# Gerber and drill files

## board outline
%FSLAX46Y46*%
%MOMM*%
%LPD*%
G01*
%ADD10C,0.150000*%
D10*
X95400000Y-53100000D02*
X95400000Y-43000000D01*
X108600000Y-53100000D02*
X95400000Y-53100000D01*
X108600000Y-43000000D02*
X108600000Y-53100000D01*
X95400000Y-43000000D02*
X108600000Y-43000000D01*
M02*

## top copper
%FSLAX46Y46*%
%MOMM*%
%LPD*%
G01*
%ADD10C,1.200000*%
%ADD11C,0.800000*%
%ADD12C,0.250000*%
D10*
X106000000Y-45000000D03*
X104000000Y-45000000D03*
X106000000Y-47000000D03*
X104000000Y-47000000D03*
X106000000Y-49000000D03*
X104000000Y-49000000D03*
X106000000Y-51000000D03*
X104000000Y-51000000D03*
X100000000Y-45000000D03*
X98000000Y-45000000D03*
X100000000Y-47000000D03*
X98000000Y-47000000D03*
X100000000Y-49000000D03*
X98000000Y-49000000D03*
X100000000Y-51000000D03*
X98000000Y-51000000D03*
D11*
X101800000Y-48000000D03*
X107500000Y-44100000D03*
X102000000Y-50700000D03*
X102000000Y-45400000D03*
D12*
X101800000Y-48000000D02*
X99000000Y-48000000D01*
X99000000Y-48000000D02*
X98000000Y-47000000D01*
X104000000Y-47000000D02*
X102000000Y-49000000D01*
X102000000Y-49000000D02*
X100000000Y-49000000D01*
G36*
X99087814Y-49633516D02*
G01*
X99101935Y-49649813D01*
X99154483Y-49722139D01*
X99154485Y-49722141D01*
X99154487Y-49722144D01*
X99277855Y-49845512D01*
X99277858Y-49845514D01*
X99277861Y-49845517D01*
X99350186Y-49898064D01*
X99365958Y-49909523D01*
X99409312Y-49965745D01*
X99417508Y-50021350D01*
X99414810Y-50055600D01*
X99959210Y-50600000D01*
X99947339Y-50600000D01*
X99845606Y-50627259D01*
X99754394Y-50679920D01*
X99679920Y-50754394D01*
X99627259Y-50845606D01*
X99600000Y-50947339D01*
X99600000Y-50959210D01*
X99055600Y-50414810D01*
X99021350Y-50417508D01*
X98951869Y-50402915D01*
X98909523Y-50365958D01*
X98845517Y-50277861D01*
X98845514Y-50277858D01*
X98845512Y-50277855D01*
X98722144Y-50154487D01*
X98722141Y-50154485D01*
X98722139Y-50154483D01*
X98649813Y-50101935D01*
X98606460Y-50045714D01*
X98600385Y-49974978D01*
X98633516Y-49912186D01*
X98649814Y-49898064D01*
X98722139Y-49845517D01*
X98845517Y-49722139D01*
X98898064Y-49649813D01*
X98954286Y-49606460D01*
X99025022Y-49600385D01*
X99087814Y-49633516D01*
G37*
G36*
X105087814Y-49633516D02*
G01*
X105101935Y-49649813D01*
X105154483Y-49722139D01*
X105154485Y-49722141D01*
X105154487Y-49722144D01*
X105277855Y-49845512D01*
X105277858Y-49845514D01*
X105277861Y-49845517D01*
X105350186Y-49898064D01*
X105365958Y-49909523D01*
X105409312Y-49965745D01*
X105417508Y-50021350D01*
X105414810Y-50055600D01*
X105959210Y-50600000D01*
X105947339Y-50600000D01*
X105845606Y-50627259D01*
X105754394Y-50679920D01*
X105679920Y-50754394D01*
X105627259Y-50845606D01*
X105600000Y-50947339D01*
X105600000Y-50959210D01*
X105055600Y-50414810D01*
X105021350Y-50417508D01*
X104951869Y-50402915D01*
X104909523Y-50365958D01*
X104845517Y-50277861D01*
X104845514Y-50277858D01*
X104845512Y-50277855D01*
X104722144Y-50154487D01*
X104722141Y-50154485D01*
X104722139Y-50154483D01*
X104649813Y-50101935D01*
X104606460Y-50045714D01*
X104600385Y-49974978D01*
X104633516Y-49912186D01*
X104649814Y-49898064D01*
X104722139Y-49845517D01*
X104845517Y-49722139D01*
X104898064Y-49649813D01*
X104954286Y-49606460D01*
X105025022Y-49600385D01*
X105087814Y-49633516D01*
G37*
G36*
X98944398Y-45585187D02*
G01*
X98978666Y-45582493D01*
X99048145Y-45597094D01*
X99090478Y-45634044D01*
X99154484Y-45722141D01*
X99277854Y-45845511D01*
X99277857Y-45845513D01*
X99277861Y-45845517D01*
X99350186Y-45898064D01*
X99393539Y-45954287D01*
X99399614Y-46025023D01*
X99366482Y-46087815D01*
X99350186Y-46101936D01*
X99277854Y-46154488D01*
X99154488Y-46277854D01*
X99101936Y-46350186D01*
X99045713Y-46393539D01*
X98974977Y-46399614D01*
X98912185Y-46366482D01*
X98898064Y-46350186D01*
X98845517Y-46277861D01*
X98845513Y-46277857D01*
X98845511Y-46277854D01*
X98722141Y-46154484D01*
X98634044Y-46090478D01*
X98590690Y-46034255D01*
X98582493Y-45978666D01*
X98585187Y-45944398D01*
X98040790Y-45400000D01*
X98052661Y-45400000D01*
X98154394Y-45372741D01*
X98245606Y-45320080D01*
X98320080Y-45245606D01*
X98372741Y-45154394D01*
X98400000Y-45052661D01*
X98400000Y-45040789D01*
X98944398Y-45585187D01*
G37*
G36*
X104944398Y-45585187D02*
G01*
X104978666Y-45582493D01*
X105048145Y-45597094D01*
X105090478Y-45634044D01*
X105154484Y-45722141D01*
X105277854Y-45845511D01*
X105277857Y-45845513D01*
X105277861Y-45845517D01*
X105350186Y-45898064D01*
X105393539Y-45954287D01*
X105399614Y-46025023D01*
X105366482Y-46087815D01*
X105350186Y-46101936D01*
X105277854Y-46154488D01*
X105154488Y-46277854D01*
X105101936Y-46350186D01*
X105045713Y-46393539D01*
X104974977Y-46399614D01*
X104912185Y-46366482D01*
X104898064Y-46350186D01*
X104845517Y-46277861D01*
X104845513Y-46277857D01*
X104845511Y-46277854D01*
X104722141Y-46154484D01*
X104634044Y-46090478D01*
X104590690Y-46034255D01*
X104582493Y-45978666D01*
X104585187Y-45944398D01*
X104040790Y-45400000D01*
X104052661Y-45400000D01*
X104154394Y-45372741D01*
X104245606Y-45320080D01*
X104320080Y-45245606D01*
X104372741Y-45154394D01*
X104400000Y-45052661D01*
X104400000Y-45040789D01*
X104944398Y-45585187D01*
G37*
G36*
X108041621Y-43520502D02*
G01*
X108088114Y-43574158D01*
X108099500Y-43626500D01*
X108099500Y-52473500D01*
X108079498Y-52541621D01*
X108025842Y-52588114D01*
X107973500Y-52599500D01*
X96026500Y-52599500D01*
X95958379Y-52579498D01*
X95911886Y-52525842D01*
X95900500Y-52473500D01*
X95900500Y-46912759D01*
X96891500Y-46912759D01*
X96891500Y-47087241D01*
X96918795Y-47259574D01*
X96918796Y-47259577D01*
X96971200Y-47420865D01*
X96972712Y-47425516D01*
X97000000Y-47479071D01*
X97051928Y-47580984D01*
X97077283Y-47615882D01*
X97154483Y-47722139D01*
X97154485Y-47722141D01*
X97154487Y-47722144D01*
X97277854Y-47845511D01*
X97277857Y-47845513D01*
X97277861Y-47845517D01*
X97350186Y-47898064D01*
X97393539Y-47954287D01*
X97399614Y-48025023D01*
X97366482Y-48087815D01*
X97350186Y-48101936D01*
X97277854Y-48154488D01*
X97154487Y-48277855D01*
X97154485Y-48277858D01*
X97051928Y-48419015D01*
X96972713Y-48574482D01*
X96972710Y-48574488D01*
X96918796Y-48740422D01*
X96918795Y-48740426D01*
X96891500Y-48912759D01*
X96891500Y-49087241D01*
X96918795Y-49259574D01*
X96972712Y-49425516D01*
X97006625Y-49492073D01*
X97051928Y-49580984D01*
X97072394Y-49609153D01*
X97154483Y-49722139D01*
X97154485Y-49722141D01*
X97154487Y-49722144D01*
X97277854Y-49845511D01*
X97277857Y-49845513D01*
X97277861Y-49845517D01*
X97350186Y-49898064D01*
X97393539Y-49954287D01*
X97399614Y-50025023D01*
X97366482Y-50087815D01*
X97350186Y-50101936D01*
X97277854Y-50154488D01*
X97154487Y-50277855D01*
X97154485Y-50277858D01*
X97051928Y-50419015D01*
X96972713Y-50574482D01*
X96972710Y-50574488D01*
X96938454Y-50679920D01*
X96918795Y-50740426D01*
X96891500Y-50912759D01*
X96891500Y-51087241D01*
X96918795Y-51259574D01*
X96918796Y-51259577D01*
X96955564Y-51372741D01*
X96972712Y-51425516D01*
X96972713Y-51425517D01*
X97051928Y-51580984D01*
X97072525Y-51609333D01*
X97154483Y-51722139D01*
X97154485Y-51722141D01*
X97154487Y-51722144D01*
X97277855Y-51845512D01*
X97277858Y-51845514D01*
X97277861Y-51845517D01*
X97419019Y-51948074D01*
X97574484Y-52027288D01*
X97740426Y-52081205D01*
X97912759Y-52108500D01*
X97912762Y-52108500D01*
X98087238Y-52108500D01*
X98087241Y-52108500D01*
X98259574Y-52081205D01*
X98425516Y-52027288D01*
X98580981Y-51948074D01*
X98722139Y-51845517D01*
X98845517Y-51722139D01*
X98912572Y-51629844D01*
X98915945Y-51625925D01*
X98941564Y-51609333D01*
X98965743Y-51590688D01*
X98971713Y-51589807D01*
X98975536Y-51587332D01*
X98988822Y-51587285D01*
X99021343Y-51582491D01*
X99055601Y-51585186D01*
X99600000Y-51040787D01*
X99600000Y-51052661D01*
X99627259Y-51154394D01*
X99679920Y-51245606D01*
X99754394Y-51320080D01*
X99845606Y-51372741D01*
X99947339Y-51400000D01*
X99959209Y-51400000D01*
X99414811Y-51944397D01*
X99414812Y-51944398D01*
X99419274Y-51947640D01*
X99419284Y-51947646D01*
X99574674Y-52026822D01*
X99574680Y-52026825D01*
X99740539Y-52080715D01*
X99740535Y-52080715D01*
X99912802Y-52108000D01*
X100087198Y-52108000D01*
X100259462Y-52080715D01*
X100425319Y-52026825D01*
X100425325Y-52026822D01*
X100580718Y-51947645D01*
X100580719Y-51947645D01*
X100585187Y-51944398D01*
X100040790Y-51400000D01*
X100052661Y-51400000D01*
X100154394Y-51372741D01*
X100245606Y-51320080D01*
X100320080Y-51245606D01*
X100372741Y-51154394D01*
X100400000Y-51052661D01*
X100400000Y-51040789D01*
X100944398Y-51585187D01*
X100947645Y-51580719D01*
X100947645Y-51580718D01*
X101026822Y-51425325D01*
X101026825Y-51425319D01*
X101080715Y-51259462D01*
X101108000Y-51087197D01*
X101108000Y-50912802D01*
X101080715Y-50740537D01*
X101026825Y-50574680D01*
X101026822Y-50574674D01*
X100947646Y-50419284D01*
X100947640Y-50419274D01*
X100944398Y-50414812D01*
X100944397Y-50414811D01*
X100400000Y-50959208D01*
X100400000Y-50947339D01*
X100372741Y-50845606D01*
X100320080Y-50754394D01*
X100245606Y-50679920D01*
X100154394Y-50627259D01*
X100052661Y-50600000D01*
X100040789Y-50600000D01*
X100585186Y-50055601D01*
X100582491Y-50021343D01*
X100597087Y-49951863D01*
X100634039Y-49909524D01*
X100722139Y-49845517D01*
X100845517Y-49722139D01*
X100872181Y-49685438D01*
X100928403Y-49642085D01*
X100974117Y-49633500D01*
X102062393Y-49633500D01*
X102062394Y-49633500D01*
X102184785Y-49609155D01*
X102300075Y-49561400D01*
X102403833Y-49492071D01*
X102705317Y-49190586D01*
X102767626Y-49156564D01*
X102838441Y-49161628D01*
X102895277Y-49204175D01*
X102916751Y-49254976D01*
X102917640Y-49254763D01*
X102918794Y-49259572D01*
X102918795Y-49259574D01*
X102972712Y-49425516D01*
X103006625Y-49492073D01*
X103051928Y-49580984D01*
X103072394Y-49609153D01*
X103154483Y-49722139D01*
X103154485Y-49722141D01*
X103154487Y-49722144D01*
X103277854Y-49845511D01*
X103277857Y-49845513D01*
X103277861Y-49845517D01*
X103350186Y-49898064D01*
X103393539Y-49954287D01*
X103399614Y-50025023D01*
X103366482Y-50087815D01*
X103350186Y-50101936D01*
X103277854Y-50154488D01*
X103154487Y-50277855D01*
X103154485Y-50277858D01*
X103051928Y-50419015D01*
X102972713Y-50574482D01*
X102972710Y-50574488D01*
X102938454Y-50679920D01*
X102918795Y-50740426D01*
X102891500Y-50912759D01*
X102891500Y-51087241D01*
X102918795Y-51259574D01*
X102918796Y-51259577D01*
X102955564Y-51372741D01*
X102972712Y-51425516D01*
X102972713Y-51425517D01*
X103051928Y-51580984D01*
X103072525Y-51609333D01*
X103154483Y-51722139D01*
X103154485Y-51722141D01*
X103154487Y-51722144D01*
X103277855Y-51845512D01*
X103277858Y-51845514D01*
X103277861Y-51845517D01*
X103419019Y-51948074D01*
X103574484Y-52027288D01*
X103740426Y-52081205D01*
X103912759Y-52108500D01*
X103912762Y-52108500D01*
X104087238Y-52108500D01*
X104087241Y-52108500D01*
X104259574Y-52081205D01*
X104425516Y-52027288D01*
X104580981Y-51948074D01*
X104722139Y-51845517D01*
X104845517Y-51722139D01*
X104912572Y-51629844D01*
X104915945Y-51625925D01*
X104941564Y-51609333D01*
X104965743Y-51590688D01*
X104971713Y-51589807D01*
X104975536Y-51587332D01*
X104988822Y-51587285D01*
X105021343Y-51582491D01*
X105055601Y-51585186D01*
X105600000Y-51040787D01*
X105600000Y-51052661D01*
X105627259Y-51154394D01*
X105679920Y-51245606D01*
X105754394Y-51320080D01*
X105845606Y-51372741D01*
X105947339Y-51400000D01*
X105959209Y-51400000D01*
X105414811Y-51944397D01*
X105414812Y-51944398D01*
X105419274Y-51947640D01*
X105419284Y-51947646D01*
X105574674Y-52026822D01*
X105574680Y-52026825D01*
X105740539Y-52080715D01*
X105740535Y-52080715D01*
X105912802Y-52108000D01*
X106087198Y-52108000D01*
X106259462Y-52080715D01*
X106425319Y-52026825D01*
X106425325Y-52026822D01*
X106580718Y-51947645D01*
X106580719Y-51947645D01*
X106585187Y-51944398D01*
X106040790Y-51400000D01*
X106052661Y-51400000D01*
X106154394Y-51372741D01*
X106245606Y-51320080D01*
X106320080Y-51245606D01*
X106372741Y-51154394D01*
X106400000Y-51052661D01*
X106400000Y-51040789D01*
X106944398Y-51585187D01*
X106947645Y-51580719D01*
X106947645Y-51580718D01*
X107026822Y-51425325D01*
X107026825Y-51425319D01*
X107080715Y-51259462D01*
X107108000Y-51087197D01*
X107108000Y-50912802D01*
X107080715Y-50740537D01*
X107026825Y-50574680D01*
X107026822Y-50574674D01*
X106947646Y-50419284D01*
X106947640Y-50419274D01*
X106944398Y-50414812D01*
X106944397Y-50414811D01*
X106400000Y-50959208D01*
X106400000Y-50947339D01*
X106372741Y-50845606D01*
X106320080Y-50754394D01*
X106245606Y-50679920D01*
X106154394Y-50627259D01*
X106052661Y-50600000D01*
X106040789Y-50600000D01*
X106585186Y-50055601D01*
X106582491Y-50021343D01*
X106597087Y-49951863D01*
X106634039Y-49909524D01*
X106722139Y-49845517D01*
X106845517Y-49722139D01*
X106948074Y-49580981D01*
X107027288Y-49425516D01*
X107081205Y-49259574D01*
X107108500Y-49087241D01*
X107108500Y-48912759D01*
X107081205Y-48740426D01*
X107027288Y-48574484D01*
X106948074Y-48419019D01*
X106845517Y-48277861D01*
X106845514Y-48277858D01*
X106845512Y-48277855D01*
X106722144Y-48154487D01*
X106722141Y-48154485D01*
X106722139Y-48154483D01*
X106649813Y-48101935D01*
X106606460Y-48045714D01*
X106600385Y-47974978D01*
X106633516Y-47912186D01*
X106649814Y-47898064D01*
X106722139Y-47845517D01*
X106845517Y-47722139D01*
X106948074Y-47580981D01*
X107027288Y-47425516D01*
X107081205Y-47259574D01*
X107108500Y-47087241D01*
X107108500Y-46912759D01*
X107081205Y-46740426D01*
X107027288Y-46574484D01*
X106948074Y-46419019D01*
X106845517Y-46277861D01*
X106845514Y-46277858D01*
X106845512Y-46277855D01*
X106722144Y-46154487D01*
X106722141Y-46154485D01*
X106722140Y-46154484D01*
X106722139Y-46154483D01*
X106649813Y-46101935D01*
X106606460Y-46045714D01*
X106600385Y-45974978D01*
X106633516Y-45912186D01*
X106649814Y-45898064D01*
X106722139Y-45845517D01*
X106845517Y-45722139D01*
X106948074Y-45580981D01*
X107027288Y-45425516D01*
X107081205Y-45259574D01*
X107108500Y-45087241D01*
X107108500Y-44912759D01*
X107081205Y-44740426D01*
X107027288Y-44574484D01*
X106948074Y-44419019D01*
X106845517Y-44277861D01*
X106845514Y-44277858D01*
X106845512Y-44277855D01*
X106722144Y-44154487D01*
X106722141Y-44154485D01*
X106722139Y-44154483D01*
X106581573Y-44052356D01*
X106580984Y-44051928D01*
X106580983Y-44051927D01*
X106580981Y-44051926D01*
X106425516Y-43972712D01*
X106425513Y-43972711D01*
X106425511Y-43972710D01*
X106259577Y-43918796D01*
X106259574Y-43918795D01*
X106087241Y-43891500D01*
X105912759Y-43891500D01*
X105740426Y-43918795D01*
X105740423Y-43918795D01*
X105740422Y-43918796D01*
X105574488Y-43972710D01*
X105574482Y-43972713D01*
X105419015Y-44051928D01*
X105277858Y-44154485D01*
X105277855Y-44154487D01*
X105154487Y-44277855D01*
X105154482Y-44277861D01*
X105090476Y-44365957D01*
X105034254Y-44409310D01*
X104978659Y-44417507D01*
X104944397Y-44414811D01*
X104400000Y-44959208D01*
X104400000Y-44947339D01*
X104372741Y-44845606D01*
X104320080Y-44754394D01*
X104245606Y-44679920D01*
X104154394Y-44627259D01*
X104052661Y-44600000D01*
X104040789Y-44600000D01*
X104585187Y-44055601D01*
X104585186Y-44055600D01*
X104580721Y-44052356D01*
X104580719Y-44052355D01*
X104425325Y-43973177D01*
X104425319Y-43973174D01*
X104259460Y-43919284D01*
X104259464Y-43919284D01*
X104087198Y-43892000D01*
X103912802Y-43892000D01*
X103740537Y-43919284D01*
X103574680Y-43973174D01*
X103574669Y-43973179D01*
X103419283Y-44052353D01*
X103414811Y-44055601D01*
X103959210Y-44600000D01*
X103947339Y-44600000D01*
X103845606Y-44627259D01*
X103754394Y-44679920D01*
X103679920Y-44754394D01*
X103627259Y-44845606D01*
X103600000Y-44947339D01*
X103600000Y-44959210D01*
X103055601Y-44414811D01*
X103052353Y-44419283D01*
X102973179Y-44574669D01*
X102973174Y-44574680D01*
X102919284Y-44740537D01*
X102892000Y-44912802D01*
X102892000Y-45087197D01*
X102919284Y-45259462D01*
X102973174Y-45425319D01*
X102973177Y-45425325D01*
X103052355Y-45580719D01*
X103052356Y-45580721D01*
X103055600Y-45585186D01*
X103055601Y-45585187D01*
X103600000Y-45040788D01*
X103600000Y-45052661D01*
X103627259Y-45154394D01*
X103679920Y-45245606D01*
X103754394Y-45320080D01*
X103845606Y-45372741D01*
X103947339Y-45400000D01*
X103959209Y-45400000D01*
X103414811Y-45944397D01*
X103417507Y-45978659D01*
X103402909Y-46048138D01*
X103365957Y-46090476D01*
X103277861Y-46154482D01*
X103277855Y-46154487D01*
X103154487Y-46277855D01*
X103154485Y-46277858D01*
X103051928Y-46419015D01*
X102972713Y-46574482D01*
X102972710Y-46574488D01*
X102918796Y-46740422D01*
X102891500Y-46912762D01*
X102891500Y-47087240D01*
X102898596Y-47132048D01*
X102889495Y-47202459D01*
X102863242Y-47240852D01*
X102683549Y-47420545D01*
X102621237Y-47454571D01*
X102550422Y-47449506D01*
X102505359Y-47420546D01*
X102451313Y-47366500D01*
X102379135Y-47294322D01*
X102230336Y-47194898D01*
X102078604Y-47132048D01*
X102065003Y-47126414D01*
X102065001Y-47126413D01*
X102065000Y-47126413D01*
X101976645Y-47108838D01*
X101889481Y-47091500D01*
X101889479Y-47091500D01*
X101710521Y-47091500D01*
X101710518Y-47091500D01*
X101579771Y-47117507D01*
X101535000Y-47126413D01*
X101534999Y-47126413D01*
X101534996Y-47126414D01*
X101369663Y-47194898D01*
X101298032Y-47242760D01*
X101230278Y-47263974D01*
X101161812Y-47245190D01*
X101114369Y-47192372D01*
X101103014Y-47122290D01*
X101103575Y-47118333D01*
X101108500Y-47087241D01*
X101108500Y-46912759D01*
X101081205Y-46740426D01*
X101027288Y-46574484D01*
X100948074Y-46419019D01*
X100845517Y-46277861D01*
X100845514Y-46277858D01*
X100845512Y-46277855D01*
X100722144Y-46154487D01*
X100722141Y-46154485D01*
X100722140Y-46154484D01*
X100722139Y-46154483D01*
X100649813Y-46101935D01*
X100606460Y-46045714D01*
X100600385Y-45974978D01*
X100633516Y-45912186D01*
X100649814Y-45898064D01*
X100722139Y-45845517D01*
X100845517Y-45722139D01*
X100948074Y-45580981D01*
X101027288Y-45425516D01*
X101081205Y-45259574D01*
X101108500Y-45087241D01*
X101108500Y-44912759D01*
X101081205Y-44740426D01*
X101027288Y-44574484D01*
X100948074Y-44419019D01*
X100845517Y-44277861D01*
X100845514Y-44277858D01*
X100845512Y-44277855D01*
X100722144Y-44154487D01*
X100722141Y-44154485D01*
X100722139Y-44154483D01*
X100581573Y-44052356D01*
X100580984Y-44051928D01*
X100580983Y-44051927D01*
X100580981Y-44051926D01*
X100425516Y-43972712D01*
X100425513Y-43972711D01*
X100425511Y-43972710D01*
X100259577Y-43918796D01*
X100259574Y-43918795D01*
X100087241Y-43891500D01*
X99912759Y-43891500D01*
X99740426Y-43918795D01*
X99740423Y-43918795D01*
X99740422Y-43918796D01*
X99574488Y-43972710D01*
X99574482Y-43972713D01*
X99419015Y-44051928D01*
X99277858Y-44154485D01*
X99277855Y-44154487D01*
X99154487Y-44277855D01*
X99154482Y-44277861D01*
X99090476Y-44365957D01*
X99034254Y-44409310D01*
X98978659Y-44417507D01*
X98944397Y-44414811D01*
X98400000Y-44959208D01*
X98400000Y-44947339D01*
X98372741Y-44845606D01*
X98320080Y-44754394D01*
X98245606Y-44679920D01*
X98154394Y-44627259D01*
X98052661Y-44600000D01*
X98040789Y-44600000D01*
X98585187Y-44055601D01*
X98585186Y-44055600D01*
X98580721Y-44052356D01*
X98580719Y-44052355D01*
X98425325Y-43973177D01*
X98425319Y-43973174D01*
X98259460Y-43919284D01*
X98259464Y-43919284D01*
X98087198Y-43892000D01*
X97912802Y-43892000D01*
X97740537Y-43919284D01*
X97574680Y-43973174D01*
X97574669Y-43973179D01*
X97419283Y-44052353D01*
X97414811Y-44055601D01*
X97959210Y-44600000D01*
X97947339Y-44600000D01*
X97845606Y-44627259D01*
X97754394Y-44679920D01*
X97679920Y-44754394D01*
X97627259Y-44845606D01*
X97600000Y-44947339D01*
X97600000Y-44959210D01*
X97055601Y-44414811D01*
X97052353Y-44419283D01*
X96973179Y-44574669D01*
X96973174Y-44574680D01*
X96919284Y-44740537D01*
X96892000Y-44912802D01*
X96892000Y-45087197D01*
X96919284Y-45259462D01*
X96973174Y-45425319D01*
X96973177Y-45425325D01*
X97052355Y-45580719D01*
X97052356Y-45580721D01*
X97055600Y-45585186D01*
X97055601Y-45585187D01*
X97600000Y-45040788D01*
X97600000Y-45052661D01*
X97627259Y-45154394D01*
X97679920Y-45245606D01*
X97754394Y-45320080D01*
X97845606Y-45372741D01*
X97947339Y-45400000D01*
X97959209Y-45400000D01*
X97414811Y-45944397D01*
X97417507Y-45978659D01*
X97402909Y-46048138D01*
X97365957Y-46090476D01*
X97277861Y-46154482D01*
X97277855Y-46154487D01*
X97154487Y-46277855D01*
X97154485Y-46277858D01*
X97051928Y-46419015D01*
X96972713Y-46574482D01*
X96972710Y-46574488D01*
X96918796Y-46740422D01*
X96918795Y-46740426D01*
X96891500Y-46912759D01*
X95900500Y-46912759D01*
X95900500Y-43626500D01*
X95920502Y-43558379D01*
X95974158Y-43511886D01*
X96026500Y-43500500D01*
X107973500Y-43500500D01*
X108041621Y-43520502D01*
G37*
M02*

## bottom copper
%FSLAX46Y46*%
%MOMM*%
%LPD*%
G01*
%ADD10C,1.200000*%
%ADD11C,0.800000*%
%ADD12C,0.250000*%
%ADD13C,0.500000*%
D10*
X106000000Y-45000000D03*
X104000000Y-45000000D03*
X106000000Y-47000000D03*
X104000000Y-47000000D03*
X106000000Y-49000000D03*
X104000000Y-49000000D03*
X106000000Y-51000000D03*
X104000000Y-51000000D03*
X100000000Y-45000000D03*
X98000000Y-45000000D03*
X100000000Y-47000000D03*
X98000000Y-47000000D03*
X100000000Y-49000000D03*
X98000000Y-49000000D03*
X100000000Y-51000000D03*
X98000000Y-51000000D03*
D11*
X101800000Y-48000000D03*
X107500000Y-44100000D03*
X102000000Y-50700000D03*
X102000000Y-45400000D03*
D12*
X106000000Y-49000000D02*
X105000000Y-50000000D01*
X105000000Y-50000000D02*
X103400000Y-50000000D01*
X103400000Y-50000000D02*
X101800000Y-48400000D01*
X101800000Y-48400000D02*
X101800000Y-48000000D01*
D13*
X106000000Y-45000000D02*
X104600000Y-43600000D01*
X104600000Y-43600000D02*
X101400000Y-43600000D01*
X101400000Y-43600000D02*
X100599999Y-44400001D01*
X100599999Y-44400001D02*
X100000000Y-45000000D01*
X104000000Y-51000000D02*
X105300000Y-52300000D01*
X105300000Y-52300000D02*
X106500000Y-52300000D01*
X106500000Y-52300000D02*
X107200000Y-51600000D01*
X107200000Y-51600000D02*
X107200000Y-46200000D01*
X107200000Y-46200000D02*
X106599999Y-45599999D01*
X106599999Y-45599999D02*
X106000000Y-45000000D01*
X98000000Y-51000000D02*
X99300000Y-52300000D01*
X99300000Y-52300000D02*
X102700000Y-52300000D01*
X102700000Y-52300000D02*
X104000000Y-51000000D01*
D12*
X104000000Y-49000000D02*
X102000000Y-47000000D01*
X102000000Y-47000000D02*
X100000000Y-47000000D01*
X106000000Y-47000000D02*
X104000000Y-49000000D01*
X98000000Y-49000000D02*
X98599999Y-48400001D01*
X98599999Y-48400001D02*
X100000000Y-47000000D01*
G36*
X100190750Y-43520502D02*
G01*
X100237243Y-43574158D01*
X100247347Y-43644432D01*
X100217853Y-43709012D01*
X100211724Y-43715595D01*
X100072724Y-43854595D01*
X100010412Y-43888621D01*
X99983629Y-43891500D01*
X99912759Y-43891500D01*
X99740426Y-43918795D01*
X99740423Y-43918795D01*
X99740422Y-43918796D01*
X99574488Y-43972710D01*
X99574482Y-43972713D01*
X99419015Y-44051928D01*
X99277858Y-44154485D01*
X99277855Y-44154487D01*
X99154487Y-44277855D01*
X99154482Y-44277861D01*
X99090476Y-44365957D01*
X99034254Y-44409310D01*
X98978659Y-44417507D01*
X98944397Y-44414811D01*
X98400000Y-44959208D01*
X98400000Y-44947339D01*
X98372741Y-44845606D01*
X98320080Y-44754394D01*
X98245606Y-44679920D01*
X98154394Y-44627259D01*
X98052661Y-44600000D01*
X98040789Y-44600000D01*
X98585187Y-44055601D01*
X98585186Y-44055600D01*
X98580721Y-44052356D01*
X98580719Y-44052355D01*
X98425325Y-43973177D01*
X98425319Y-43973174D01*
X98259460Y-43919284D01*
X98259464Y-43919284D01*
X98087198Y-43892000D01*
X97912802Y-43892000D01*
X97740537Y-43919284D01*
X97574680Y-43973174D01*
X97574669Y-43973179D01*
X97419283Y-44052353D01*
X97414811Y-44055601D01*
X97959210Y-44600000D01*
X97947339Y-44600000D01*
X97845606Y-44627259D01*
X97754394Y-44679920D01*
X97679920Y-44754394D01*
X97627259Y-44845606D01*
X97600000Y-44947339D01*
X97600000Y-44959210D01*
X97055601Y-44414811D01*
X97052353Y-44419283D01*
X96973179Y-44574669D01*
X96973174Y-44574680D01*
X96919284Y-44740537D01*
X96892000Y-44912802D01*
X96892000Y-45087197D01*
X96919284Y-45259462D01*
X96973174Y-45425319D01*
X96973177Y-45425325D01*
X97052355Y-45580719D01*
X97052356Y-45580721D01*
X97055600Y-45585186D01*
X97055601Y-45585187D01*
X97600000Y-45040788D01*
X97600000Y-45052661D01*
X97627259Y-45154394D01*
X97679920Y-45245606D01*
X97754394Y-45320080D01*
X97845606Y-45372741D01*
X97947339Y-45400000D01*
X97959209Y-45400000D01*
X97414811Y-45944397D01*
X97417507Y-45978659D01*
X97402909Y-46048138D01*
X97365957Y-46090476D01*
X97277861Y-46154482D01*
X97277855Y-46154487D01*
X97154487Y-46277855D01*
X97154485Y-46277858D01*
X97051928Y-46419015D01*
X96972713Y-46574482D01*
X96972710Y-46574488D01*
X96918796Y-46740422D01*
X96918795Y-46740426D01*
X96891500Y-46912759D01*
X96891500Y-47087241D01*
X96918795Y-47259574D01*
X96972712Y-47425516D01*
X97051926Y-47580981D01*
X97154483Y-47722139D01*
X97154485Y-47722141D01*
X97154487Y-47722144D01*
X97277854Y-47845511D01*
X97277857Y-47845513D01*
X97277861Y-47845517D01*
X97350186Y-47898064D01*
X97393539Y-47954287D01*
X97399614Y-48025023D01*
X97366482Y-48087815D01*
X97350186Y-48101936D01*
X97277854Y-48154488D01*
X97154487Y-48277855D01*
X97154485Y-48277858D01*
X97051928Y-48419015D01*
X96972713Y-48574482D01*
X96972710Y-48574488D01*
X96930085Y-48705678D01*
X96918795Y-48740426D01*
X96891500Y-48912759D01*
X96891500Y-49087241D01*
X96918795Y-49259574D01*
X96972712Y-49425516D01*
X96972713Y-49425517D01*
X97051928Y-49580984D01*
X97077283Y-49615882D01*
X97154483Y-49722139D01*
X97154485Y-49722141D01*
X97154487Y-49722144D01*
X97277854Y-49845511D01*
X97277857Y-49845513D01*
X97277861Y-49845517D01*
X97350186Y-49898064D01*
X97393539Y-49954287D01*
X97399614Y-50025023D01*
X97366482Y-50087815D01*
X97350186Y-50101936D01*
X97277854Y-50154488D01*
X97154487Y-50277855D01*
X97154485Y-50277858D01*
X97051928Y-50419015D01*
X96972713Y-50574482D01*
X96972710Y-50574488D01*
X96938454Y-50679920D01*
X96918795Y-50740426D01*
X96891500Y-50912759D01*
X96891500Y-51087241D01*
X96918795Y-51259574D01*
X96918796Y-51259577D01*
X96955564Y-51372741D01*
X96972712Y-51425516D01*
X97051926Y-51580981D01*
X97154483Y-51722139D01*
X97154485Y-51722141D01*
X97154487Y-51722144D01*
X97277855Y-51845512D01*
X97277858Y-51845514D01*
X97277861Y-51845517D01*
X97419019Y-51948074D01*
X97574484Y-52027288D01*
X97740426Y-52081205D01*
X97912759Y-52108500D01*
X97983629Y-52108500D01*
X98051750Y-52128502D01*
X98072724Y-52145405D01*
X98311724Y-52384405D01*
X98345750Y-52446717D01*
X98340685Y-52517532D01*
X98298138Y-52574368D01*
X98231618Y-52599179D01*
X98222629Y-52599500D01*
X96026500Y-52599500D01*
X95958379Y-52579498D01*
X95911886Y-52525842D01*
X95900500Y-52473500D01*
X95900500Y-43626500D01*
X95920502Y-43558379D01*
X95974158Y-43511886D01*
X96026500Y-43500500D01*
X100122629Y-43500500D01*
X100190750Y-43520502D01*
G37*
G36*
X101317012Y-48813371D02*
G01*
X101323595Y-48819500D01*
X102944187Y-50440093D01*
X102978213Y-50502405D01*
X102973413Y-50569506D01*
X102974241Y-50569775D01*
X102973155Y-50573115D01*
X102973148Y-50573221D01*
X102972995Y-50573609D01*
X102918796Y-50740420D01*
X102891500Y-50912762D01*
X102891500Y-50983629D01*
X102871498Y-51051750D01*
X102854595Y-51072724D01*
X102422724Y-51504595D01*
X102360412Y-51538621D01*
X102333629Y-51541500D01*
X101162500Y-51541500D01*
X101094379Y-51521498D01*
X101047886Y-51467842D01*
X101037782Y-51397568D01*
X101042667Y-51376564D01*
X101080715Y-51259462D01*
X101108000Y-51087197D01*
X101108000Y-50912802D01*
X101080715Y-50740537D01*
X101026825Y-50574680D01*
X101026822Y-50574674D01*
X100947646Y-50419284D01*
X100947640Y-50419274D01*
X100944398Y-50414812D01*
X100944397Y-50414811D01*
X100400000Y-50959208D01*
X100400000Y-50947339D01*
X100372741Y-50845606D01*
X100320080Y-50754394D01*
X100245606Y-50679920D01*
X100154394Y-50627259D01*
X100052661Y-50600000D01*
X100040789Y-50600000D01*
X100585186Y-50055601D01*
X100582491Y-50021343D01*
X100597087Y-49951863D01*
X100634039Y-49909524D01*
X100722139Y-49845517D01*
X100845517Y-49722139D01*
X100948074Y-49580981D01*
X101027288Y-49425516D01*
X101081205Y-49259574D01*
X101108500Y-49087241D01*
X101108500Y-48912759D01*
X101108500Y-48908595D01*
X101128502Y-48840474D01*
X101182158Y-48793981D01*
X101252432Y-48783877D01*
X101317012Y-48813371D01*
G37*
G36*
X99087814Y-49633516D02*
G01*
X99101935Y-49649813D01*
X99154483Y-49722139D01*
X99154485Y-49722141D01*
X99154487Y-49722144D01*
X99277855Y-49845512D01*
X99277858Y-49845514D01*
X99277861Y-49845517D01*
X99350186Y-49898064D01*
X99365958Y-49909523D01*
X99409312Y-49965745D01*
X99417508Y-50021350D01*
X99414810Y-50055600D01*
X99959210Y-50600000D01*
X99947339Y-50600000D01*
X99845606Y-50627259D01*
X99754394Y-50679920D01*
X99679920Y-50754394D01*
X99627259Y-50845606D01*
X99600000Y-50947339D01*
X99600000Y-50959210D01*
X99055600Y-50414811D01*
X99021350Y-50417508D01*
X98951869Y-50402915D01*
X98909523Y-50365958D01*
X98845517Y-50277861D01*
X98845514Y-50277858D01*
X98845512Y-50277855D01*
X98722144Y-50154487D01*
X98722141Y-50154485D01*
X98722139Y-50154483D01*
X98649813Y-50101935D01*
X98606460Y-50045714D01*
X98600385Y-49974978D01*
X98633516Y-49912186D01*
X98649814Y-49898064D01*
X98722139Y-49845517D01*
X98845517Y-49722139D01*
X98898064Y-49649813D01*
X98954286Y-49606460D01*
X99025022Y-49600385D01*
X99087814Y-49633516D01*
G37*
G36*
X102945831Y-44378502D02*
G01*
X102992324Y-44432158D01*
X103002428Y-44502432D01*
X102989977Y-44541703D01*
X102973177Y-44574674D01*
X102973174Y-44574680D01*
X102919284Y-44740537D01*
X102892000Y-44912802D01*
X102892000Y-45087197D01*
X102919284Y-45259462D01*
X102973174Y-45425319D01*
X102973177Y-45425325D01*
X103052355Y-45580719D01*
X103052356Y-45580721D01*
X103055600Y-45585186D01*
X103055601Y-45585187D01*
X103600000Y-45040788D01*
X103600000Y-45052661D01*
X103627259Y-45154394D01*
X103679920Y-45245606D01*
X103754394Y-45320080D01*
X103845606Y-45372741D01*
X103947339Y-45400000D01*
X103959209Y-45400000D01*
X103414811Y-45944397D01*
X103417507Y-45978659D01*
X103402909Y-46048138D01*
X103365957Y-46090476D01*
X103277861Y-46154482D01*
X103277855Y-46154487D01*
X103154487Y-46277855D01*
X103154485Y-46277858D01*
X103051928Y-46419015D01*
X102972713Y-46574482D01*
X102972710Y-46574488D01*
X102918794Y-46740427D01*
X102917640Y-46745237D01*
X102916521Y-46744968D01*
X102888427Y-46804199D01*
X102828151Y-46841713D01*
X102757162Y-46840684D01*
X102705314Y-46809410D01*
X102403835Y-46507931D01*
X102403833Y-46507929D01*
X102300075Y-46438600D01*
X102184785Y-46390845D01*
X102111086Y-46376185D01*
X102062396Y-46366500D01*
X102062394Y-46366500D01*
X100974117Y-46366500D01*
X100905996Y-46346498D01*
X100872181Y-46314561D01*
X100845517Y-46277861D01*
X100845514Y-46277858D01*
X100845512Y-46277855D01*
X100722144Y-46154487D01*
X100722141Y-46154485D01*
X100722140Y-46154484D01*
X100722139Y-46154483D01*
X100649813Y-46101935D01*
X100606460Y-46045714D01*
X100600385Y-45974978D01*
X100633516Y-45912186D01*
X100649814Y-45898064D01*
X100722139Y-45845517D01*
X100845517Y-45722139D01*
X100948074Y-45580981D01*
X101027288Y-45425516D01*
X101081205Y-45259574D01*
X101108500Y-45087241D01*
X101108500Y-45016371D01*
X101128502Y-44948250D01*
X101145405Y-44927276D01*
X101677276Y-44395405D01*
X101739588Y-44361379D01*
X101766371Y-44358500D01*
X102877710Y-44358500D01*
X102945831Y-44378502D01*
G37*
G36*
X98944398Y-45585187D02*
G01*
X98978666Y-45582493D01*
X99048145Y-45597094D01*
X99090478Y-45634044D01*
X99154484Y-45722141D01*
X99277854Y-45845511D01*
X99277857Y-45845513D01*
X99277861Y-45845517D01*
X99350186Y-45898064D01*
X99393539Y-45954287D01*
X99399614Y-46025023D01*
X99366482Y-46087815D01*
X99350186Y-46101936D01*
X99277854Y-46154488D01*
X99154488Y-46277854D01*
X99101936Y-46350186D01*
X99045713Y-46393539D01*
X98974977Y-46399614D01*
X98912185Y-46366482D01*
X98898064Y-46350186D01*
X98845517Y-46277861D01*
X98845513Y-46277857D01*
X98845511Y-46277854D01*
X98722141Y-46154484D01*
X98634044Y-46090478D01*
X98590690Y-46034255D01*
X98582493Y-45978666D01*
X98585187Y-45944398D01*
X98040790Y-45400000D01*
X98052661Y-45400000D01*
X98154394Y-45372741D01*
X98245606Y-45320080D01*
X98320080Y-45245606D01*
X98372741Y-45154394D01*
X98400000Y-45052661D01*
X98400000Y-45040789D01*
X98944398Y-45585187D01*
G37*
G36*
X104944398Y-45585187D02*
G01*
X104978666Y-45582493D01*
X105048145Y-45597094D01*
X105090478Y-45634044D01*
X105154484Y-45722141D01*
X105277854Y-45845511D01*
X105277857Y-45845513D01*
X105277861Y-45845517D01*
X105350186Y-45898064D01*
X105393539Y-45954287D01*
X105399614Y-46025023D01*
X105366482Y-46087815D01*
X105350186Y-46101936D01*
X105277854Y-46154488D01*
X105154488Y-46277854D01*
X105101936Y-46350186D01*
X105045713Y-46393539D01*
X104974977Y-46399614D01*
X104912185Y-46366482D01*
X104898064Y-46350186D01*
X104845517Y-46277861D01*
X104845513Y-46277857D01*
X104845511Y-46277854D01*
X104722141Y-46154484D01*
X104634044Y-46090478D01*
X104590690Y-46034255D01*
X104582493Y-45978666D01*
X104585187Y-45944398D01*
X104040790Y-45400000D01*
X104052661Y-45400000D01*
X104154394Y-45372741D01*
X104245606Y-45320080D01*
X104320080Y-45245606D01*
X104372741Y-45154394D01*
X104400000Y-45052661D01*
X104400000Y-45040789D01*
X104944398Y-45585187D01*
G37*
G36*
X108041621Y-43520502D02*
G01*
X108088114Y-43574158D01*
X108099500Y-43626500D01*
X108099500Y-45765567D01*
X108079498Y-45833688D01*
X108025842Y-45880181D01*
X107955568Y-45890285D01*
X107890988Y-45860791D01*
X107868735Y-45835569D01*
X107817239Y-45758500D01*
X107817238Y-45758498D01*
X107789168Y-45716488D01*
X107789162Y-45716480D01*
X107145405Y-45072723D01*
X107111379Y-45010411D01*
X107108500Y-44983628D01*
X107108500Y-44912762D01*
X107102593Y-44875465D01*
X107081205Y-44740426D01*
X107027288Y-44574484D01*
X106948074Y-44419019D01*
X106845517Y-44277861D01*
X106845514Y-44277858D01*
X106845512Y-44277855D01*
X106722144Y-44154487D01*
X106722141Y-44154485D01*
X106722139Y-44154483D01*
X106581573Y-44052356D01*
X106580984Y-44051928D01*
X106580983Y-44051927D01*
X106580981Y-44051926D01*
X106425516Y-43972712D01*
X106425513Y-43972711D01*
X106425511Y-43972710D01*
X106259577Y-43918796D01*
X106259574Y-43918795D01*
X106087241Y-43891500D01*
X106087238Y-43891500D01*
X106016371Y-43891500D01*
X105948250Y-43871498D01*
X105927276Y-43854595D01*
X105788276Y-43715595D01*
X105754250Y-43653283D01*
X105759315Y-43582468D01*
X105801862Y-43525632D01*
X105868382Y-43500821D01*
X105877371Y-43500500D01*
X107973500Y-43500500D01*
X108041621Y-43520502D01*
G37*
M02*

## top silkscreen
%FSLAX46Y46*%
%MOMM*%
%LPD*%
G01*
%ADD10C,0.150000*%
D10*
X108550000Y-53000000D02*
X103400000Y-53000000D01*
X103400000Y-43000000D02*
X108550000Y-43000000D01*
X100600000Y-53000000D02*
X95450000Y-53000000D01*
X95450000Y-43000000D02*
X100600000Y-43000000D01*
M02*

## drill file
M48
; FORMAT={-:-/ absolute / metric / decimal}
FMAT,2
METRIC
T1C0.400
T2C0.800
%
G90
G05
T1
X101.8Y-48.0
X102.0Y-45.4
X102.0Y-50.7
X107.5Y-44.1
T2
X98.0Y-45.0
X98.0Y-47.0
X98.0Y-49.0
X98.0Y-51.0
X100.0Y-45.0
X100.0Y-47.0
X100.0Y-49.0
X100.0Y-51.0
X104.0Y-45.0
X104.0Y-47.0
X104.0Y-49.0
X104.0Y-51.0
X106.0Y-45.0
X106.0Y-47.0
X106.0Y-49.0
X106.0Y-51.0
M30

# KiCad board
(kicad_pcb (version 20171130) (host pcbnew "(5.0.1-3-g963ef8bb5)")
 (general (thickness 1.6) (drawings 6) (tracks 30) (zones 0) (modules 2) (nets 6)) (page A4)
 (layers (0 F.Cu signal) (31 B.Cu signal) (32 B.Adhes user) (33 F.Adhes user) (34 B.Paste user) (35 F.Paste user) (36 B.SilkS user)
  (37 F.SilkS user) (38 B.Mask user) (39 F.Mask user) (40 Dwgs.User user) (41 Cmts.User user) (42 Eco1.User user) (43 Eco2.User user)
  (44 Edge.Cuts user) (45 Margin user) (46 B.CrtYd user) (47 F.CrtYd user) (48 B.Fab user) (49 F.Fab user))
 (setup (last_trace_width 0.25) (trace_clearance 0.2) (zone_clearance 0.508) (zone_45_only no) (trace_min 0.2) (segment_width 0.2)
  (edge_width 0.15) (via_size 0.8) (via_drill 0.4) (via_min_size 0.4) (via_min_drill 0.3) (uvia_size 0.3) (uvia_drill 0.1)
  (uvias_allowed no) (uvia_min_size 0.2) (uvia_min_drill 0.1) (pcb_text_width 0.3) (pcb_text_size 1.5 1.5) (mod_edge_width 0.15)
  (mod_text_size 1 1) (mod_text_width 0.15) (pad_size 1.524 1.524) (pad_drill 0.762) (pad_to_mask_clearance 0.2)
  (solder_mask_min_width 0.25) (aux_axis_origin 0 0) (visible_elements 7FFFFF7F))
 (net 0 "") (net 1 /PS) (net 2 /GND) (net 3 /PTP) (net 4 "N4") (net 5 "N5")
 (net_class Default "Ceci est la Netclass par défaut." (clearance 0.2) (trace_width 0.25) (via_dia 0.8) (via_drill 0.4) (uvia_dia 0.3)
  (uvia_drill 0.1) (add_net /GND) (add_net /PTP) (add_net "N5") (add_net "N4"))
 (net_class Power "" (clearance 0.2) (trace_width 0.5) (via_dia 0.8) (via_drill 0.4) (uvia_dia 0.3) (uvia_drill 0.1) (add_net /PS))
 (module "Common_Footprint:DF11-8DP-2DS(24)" (layer F.Cu) (at 105 48 270)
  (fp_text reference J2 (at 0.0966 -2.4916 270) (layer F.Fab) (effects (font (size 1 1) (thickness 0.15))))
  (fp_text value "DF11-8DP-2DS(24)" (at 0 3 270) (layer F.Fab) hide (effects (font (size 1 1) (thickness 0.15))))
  (fp_line (start 5 -3.55) (end 5 1.6) (layer F.SilkS) (width 0.15))
  (fp_line (start -5 1.6) (end -5 -3.55) (layer F.SilkS) (width 0.15))
  (pad 8 thru_hole circle (at -3 -1 270) (size 1.2 1.2) (drill 0.8) (layers *.Cu *.Mask) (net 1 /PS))
  (pad 7 thru_hole circle (at -3 1 270) (size 1.2 1.2) (drill 0.8) (layers *.Cu *.Mask) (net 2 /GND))
  (pad 6 thru_hole circle (at -1 -1 270) (size 1.2 1.2) (drill 0.8) (layers *.Cu *.Mask) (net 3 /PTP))
  (pad 5 thru_hole circle (at -1 1 270) (size 1.2 1.2) (drill 0.8) (layers *.Cu *.Mask) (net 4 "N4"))
  (pad 4 thru_hole circle (at 1 -1 270) (size 1.2 1.2) (drill 0.8) (layers *.Cu *.Mask) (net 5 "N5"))
  (pad 3 thru_hole circle (at 1 1 270) (size 1.2 1.2) (drill 0.8) (layers *.Cu *.Mask) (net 3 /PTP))
  (pad 2 thru_hole circle (at 3 -1 270) (size 1.2 1.2) (drill 0.8) (layers *.Cu *.Mask) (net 2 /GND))
  (pad 1 thru_hole circle (at 3 1 270) (size 1.2 1.2) (drill 0.8) (layers *.Cu *.Mask) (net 1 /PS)))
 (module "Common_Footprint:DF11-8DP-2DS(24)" (layer F.Cu) (at 99 48 90)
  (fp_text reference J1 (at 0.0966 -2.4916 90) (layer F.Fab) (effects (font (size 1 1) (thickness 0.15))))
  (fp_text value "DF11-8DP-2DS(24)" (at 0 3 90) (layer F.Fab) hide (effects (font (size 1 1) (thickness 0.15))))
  (fp_line (start -5 1.6) (end -5 -3.55) (layer F.SilkS) (width 0.15))
  (fp_line (start 5 -3.55) (end 5 1.6) (layer F.SilkS) (width 0.15))
  (pad 1 thru_hole circle (at 3 1 90) (size 1.2 1.2) (drill 0.8) (layers *.Cu *.Mask) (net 1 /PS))
  (pad 2 thru_hole circle (at 3 -1 90) (size 1.2 1.2) (drill 0.8) (layers *.Cu *.Mask) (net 2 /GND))
  (pad 3 thru_hole circle (at 1 1 90) (size 1.2 1.2) (drill 0.8) (layers *.Cu *.Mask) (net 3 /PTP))
  (pad 4 thru_hole circle (at 1 -1 90) (size 1.2 1.2) (drill 0.8) (layers *.Cu *.Mask) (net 5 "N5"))
  (pad 5 thru_hole circle (at -1 1 90) (size 1.2 1.2) (drill 0.8) (layers *.Cu *.Mask) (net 4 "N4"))
  (pad 6 thru_hole circle (at -1 -1 90) (size 1.2 1.2) (drill 0.8) (layers *.Cu *.Mask) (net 3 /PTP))
  (pad 7 thru_hole circle (at -3 1 90) (size 1.2 1.2) (drill 0.8) (layers *.Cu *.Mask) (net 2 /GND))
  (pad 8 thru_hole circle (at -3 -1 90) (size 1.2 1.2) (drill 0.8) (layers *.Cu *.Mask) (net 1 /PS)))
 (gr_line (start 95.4 53.1) (end 95.4 43) (layer Edge.Cuts) (width 0.15))
 (gr_line (start 108.6 53.1) (end 95.4 53.1) (layer Edge.Cuts) (width 0.15))
 (gr_line (start 108.6 43) (end 108.6 53.1) (layer Edge.Cuts) (width 0.15))
 (gr_line (start 95.4 43) (end 108.6 43) (layer Edge.Cuts) (width 0.15))
 (segment (start 106 49) (end 105 50) (width 0.25) (layer B.Cu) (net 5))
 (segment (start 105 50) (end 103.4 50) (width 0.25) (layer B.Cu) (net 5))
 (segment (start 103.4 50) (end 101.8 48.4) (width 0.25) (layer B.Cu) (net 5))
 (segment (start 101.8 48.4) (end 101.8 48) (width 0.25) (layer B.Cu) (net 5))
 (segment (start 101.8 48) (end 99 48) (width 0.25) (layer F.Cu) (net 5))
 (segment (start 99 48) (end 98 47) (width 0.25) (layer F.Cu) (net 5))
 (via (at 101.8 48) (size 0.8) (drill 0.4) (layers F.Cu B.Cu) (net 5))
 (segment (start 104 47) (end 102 49) (width 0.25) (layer F.Cu) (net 4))
 (segment (start 102 49) (end 100 49) (width 0.25) (layer F.Cu) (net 4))
 (segment (start 106 45) (end 104.6 43.6) (width 0.5) (layer B.Cu) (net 1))
 (segment (start 104.6 43.6) (end 101.4 43.6) (width 0.5) (layer B.Cu) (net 1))
 (segment (start 101.4 43.6) (end 100.599999 44.400001) (width 0.5) (layer B.Cu) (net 1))
 (segment (start 100.599999 44.400001) (end 100 45) (width 0.5) (layer B.Cu) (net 1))
 (segment (start 104 51) (end 105.3 52.3) (width 0.5) (layer B.Cu) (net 1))
 (segment (start 105.3 52.3) (end 106.5 52.3) (width 0.5) (layer B.Cu) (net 1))
 (segment (start 106.5 52.3) (end 107.2 51.6) (width 0.5) (layer B.Cu) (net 1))
 (segment (start 107.2 51.6) (end 107.2 46.2) (width 0.5) (layer B.Cu) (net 1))
 (segment (start 107.2 46.2) (end 106.599999 45.599999) (width 0.5) (layer B.Cu) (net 1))
 (segment (start 106.599999 45.599999) (end 106 45) (width 0.5) (layer B.Cu) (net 1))
 (segment (start 98 51) (end 99.3 52.3) (width 0.5) (layer B.Cu) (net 1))
 (segment (start 99.3 52.3) (end 102.7 52.3) (width 0.5) (layer B.Cu) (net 1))
 (segment (start 102.7 52.3) (end 104 51) (width 0.5) (layer B.Cu) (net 1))
 (via (at 107.5 44.1) (size 0.8) (drill 0.4) (layers F.Cu B.Cu) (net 2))
 (via (at 102 50.7) (size 0.8) (drill 0.4) (layers F.Cu B.Cu) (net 2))
 (via (at 102 45.4) (size 0.8) (drill 0.4) (layers F.Cu B.Cu) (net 2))
 (segment (start 104 49) (end 102 47) (width 0.25) (layer B.Cu) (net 3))
 (segment (start 102 47) (end 100 47) (width 0.25) (layer B.Cu) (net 3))
 (segment (start 106 47) (end 104 49) (width 0.25) (layer B.Cu) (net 3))
 (segment (start 98 49) (end 98.599999 48.400001) (width 0.25) (layer B.Cu) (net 3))
 (segment (start 98.599999 48.400001) (end 100 47) (width 0.25) (layer B.Cu) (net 3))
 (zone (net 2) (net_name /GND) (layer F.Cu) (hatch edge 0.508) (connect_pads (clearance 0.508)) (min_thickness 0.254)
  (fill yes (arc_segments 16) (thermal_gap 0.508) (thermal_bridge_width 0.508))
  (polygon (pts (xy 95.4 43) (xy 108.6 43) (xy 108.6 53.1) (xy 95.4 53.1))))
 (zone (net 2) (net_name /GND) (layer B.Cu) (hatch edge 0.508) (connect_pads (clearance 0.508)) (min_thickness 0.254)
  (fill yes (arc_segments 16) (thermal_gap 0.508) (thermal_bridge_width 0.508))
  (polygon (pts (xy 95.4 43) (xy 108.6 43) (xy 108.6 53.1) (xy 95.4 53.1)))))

